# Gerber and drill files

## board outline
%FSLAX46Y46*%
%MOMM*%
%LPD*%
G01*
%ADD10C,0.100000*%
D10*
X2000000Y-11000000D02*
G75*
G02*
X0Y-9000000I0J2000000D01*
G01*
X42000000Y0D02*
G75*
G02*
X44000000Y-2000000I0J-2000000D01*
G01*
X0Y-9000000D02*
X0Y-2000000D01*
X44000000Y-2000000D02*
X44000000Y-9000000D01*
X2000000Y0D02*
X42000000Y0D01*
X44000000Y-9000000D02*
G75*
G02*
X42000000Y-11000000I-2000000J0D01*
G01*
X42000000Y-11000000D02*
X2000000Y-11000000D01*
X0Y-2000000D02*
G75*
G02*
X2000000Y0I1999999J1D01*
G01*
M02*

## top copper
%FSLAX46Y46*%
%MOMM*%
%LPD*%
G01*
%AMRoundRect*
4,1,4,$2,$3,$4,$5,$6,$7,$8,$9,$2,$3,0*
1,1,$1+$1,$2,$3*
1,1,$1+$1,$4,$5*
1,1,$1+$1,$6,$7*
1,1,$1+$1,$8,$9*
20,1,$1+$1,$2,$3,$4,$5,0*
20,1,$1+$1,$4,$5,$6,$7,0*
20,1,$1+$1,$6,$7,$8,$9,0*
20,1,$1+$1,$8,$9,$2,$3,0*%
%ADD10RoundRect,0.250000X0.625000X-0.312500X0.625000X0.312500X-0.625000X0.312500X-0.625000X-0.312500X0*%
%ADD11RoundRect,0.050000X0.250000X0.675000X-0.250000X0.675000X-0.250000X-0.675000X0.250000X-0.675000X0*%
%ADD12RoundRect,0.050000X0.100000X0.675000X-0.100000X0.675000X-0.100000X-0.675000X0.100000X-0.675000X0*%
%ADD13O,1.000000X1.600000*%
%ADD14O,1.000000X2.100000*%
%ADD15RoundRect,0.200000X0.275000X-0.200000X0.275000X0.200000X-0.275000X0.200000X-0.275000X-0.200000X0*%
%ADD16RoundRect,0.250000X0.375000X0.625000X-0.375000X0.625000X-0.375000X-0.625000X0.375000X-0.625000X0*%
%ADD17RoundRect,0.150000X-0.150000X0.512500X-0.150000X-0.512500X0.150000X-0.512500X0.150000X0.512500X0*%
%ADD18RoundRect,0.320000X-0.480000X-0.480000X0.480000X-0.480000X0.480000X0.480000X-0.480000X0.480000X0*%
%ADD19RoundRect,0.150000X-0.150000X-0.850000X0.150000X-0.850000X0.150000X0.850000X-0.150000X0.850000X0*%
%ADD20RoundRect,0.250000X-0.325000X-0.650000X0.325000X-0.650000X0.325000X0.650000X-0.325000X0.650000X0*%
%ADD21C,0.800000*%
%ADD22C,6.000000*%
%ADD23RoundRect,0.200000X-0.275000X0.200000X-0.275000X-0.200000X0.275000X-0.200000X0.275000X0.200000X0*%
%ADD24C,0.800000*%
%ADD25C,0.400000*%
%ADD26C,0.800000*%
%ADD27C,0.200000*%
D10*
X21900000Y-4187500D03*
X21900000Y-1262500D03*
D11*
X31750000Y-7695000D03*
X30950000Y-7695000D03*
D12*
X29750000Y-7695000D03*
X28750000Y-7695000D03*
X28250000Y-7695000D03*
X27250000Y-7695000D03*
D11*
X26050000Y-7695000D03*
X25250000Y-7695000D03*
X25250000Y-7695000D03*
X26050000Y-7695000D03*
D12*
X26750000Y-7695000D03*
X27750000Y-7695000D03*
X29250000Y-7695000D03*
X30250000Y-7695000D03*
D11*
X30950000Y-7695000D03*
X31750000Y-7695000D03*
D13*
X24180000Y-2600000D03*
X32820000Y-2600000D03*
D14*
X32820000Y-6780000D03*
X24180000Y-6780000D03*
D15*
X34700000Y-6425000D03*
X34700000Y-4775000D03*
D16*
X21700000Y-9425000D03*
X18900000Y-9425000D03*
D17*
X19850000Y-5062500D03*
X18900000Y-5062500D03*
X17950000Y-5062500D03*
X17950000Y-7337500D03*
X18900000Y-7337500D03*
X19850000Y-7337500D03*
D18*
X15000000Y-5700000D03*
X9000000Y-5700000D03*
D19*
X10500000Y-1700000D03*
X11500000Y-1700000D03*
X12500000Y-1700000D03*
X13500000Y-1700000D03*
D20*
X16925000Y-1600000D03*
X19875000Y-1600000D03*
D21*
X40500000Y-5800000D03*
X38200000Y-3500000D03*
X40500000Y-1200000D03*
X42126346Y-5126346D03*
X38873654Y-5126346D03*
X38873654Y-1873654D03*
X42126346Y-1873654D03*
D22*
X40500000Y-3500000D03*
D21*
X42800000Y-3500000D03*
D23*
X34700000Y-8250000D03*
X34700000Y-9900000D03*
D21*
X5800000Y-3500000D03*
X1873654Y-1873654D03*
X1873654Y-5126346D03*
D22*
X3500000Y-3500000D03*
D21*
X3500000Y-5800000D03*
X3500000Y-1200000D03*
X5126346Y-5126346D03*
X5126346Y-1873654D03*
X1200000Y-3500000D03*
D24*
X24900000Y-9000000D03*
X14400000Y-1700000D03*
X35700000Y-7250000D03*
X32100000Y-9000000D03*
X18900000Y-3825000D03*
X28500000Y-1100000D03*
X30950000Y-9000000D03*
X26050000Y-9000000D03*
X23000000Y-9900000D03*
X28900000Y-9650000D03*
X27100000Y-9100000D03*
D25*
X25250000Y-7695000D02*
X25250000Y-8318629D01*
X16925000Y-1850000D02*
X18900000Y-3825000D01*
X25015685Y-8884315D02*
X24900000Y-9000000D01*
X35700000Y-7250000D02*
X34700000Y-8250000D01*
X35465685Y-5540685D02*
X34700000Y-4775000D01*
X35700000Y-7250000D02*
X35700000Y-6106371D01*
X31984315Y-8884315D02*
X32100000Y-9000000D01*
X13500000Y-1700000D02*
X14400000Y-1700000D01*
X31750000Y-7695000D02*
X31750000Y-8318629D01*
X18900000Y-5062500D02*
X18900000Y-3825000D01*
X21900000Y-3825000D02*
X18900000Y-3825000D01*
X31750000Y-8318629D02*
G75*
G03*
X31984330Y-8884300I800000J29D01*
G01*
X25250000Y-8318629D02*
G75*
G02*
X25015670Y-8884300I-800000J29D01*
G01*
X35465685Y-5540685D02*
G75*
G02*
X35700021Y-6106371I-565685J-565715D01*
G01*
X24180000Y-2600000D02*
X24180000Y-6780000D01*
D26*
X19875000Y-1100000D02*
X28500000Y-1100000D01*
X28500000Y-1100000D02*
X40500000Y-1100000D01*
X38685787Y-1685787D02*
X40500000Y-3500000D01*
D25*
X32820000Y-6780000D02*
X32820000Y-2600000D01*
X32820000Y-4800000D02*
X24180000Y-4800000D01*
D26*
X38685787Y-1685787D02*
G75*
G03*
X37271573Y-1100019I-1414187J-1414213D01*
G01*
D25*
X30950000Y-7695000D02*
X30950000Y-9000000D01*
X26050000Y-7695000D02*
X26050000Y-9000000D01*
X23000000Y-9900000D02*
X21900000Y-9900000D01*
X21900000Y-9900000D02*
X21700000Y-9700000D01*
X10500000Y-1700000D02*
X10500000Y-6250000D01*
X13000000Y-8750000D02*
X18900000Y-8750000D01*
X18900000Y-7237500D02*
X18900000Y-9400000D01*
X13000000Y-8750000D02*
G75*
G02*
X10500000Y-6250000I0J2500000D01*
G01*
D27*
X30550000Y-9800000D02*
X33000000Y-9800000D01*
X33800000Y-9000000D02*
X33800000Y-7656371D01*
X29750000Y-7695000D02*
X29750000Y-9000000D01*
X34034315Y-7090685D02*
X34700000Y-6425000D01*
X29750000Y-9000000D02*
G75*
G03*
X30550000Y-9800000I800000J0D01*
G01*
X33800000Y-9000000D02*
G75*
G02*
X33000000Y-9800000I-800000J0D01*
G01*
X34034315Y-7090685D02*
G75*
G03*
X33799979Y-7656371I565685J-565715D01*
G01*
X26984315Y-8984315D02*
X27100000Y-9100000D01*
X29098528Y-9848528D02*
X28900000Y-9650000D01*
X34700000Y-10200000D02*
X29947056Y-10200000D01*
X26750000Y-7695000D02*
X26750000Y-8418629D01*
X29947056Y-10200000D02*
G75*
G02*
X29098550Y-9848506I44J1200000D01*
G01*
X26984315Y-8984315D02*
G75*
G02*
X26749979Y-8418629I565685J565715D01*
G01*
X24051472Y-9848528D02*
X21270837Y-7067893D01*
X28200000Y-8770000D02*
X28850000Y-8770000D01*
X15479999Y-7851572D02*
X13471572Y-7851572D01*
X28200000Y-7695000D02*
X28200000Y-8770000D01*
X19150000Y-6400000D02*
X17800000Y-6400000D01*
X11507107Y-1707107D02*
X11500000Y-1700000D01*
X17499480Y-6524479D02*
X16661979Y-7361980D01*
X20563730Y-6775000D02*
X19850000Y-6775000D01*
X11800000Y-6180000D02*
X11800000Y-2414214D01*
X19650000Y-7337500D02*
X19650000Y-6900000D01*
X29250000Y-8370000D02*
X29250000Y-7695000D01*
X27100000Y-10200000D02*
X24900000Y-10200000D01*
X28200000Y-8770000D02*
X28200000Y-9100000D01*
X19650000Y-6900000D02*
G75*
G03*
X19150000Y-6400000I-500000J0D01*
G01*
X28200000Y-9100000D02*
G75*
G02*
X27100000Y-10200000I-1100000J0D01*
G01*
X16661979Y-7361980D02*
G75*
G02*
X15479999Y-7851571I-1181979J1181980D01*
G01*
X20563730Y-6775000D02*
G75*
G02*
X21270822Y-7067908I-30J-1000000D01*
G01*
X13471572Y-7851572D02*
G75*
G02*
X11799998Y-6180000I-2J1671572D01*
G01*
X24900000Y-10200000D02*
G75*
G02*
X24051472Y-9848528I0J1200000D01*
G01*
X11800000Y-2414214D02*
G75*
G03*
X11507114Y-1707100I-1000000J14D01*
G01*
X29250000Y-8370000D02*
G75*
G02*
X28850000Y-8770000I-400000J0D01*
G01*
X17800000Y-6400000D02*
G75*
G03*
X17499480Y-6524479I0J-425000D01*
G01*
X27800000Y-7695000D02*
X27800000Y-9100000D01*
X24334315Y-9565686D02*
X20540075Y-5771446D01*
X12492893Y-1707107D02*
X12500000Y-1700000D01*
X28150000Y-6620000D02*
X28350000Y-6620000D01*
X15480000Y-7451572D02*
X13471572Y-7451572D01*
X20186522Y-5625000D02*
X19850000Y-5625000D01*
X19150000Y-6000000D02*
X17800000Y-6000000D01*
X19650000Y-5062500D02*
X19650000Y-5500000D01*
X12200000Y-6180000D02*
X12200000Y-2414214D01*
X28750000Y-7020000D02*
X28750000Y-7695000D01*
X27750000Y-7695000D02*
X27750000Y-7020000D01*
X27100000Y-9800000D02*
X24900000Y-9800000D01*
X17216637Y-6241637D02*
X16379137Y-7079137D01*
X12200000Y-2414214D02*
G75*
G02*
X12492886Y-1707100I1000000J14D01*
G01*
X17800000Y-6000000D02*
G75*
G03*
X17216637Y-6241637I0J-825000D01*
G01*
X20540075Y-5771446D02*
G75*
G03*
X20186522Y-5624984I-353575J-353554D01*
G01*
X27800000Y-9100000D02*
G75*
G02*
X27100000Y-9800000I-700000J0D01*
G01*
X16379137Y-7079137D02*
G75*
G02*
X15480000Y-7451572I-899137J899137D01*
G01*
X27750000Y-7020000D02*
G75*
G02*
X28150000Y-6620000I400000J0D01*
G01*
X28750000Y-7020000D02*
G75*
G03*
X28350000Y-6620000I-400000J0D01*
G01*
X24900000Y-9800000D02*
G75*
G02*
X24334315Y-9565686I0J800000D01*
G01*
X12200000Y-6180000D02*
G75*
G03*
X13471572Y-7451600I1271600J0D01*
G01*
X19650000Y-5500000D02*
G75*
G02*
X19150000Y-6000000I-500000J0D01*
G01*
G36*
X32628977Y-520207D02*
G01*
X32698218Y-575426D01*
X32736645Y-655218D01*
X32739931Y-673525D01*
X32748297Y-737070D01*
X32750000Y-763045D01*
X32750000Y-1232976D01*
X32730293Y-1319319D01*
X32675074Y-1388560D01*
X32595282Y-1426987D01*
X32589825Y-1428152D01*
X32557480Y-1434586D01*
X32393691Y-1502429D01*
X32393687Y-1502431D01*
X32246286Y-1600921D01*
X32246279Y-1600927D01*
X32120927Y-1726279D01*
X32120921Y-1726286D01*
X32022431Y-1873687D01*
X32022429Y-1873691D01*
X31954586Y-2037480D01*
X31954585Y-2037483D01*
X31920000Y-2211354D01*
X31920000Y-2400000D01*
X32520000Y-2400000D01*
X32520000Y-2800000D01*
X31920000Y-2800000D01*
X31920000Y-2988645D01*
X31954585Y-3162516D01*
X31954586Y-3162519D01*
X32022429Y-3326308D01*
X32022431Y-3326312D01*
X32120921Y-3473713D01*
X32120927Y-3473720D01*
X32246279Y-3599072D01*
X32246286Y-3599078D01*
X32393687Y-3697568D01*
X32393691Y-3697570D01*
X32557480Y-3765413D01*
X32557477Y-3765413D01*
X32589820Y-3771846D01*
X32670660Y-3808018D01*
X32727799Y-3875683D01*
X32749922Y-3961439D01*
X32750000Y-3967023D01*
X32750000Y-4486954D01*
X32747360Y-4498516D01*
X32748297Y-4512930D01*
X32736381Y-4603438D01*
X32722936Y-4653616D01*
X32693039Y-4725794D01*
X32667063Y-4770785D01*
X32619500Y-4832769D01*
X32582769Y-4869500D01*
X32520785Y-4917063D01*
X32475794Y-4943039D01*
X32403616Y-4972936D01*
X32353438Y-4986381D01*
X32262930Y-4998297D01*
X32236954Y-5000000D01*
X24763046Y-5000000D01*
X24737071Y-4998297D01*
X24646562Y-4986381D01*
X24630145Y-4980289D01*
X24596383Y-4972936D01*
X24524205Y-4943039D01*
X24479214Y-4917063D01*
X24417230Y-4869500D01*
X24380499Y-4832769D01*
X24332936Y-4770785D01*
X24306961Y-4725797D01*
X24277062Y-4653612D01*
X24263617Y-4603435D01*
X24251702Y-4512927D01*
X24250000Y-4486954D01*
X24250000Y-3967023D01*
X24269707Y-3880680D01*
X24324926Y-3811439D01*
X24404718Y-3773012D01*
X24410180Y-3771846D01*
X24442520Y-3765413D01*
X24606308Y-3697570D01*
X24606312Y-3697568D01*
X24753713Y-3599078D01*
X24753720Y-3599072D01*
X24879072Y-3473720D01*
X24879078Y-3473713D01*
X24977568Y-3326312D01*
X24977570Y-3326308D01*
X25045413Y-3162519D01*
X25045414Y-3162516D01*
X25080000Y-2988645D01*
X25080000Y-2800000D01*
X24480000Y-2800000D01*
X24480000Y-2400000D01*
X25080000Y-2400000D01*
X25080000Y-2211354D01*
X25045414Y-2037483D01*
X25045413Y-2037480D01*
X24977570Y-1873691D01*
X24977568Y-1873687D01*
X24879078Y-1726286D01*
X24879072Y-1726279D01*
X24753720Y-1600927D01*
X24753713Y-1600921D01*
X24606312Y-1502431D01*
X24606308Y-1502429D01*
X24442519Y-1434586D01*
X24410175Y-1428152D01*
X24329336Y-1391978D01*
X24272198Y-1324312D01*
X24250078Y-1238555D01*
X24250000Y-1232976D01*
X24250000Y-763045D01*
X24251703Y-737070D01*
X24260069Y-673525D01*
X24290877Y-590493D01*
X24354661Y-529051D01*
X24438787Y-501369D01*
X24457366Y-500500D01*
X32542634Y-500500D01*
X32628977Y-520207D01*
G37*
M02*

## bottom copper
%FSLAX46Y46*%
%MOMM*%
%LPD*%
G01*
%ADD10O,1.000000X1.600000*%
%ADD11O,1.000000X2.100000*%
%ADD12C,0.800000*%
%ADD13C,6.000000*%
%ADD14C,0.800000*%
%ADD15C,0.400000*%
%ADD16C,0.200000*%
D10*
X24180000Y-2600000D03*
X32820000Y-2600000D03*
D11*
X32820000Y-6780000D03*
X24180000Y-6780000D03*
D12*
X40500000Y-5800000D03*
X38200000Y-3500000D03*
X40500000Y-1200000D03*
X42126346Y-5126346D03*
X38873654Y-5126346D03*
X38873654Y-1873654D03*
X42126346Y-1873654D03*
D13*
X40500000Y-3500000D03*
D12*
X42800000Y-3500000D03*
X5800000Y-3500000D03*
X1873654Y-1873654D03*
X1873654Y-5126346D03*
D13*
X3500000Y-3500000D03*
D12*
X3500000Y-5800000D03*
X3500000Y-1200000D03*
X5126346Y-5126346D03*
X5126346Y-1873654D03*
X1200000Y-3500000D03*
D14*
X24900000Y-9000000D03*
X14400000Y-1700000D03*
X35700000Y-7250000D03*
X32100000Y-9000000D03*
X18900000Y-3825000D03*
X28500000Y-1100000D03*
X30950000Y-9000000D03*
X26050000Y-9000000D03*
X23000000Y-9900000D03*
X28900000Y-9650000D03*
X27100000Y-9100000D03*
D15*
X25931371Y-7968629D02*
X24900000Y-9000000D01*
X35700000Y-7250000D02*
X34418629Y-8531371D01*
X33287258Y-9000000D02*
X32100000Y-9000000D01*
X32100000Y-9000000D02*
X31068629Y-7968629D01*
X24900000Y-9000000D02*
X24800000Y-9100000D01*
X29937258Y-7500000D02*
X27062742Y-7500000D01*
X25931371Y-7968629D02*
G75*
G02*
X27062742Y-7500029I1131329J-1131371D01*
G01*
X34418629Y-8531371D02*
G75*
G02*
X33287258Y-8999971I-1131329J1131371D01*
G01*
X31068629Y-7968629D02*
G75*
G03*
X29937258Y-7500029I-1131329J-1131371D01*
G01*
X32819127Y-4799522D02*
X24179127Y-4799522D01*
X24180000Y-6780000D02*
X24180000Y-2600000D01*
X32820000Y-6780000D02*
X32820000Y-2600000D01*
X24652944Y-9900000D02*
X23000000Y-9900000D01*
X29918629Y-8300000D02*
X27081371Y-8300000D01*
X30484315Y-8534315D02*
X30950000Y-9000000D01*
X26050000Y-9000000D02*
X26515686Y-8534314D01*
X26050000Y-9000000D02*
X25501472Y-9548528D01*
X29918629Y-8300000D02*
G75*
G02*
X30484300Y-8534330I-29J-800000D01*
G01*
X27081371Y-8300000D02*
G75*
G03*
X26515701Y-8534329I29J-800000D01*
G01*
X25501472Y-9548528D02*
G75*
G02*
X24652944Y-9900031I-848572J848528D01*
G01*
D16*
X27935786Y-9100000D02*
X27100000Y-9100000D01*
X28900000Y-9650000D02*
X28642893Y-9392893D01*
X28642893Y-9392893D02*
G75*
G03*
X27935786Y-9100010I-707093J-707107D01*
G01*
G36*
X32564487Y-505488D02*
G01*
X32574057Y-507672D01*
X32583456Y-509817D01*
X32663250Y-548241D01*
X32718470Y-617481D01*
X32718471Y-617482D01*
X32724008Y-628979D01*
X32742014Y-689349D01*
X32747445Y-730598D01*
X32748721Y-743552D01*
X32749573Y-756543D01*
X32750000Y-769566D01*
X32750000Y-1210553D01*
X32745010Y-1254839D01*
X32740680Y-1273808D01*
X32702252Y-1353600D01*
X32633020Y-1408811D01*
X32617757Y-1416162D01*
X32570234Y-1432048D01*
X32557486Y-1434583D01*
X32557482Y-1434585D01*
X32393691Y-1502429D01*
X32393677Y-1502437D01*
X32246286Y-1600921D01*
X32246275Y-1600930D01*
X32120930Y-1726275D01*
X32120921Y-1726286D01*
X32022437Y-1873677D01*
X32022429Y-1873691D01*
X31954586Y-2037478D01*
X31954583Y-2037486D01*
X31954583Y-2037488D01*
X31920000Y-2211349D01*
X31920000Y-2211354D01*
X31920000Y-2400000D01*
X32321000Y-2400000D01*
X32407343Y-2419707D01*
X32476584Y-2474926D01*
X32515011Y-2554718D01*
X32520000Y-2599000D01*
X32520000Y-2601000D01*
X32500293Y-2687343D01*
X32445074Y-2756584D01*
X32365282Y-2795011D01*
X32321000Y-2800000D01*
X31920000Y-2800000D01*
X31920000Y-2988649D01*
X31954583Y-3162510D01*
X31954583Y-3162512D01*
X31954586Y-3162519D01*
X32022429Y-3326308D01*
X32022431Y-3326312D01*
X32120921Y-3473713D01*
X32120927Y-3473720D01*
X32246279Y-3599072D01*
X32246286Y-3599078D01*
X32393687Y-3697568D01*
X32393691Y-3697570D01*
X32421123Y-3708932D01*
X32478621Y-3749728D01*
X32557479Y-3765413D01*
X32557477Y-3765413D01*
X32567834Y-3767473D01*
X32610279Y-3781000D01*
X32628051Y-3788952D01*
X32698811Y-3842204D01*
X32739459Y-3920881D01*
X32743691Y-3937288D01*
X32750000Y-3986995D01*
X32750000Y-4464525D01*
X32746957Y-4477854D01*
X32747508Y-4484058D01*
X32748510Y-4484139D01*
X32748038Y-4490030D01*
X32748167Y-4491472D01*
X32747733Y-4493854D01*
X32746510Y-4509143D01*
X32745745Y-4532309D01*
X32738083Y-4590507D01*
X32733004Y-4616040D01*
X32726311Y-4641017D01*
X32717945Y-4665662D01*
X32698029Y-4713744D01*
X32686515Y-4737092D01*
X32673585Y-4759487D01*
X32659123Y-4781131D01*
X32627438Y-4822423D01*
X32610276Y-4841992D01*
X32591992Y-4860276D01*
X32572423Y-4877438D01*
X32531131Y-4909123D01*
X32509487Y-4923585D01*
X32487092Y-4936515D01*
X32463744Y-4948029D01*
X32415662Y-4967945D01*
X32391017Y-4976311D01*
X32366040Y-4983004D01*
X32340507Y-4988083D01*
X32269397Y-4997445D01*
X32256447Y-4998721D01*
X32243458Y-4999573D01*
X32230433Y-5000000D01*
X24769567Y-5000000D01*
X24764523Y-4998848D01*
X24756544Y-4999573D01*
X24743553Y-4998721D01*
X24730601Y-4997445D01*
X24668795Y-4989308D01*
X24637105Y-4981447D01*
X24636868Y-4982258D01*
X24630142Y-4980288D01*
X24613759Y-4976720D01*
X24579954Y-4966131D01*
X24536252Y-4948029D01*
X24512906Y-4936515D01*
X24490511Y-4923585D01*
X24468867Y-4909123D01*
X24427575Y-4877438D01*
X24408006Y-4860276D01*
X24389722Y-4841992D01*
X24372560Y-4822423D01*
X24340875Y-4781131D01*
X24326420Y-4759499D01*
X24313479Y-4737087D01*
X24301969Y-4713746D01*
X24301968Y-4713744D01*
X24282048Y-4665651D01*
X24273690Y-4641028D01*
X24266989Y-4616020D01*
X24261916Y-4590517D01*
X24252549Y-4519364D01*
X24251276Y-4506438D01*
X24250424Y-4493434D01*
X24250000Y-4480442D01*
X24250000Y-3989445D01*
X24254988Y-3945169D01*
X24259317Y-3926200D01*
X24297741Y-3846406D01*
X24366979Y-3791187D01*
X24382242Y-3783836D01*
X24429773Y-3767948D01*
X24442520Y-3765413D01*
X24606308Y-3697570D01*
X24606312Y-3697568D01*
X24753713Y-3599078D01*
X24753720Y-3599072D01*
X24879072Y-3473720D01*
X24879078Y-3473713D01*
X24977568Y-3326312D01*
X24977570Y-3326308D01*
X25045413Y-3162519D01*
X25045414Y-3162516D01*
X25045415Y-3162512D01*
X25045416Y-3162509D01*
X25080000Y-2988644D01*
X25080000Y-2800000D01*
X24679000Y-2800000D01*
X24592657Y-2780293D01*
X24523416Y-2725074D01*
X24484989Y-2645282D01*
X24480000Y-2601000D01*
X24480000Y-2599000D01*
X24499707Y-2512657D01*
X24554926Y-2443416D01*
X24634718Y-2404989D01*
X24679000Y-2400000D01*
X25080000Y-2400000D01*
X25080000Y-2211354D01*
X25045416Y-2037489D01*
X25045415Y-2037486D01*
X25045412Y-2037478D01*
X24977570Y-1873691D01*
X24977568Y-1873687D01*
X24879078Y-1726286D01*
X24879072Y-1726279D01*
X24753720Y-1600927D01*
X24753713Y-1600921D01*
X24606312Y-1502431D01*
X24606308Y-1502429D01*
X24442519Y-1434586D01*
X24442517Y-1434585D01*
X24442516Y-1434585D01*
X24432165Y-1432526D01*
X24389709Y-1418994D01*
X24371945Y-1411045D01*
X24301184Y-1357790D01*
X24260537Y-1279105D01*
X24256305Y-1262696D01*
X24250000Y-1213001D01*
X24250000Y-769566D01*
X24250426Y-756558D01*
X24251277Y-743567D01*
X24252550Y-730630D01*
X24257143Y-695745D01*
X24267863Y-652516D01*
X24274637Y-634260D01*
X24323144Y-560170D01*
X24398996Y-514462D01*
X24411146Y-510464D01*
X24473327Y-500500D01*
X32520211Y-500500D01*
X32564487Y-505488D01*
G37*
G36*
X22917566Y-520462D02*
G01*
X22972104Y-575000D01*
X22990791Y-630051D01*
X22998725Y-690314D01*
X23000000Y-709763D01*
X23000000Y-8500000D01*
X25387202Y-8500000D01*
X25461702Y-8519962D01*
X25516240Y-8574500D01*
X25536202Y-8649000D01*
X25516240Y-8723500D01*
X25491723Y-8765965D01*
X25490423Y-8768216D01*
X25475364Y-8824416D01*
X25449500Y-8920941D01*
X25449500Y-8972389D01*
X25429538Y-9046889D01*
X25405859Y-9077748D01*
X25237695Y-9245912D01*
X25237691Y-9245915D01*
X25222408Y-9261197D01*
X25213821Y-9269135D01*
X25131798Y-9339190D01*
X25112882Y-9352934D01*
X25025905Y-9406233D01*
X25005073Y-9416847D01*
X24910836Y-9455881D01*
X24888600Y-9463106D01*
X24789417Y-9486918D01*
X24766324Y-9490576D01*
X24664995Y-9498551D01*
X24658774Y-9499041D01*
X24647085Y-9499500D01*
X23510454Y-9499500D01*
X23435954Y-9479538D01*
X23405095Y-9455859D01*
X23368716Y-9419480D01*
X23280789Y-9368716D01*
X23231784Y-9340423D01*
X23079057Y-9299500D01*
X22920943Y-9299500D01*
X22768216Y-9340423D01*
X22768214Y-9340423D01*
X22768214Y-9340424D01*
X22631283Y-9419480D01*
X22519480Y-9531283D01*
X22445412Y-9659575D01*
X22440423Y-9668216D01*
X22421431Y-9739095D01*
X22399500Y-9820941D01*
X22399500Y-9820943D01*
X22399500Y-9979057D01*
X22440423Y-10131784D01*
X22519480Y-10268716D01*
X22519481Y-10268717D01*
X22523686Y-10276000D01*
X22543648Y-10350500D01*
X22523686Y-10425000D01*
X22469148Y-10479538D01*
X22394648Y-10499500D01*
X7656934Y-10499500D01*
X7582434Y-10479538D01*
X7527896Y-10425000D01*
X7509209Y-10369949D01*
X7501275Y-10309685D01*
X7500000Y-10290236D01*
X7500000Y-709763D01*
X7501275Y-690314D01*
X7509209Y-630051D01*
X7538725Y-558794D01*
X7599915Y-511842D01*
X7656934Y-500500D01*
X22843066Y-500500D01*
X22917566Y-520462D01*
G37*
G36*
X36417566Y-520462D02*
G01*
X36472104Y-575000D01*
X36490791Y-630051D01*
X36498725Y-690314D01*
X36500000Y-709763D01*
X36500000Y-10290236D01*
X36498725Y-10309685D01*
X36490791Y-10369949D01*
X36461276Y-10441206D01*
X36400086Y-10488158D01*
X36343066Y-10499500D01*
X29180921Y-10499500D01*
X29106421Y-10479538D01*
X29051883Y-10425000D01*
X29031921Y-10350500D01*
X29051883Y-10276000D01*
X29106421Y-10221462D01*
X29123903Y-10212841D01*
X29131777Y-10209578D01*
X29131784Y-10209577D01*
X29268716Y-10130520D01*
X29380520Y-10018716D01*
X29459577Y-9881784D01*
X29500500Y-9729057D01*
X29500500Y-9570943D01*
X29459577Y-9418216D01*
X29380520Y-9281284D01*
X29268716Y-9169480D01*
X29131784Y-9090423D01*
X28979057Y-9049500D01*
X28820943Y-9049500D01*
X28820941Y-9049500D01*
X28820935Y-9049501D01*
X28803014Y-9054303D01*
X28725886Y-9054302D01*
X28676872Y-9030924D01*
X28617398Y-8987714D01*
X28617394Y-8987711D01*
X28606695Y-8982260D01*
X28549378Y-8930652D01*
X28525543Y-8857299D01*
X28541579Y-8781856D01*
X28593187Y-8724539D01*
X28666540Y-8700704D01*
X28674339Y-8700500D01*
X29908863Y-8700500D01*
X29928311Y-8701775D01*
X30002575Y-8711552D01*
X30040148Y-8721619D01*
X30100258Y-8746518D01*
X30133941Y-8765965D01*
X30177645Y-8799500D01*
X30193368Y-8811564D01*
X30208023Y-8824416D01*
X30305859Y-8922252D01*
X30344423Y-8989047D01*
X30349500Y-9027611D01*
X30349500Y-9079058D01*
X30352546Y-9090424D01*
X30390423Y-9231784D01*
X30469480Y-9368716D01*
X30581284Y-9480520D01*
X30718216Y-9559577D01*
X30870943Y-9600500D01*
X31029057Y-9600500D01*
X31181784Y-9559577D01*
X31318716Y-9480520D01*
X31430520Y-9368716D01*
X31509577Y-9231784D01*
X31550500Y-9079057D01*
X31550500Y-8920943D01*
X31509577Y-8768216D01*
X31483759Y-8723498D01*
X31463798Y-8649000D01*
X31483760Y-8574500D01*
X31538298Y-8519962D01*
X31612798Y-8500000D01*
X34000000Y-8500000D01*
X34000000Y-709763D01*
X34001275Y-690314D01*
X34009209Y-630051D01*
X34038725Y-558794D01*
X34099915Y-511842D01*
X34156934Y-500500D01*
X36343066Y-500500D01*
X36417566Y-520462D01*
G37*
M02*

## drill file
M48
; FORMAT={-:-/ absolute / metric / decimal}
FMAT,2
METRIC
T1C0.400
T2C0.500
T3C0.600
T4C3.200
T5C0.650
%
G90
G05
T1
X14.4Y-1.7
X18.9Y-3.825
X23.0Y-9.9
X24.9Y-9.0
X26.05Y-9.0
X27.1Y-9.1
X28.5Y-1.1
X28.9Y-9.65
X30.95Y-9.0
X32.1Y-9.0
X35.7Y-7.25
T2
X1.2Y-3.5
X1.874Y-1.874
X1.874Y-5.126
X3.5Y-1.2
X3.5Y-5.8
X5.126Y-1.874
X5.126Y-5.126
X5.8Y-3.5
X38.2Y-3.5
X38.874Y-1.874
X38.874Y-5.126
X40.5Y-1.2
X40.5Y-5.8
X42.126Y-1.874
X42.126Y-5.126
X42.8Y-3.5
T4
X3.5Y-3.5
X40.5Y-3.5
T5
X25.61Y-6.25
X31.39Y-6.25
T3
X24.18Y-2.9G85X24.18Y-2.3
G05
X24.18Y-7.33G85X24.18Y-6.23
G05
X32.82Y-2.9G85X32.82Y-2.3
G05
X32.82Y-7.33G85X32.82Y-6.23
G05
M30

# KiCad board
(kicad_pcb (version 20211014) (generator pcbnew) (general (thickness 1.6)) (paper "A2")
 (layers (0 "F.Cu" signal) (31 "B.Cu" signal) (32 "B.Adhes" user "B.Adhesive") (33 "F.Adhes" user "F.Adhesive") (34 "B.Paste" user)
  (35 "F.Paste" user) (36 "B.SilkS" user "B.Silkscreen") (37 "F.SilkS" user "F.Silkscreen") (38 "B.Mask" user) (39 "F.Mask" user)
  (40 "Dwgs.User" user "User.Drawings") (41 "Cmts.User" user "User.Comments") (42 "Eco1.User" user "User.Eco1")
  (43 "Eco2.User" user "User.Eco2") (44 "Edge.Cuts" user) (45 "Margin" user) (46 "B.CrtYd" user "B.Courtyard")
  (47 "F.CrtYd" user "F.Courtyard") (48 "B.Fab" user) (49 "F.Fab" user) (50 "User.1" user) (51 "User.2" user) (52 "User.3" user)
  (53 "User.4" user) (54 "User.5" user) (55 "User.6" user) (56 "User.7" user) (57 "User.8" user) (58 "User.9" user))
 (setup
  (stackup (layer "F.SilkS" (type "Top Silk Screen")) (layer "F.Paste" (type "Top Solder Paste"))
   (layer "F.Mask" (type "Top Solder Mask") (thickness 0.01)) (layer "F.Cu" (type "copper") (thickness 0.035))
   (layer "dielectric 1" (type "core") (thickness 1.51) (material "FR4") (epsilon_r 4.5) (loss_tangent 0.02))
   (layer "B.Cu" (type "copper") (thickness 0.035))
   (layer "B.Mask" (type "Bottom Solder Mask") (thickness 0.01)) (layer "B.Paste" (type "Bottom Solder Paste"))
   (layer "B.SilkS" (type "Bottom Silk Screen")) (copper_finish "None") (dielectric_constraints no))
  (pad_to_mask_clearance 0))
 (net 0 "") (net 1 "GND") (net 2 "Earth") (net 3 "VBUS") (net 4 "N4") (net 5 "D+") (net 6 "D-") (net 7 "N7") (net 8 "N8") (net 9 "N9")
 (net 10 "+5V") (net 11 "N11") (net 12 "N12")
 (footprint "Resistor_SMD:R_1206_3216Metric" (layer "F.Cu") (at 21.9 2.725 90)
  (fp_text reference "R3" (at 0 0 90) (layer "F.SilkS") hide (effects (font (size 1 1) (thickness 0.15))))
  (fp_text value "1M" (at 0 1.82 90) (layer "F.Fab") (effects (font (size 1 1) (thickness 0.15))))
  (pad "1" smd roundrect (at -1.4625 0 90) (size 1.125 1.75) (layers "F.Cu" "F.Paste" "F.Mask") (roundrect_rratio 0.2222222222)
   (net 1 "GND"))
  (pad "2" smd roundrect (at 1.4625 0 90) (size 1.125 1.75) (layers "F.Cu" "F.Paste" "F.Mask") (roundrect_rratio 0.2222222222)
   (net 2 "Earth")))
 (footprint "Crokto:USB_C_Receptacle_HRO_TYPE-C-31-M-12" (layer "F.Cu") (at 28.5 3.65 180)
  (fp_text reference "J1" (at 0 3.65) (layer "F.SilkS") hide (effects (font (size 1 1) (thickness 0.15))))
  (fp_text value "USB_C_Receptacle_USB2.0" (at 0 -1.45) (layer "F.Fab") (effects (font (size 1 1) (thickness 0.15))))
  (pad "" np_thru_hole circle (at -2.89 -2.6 180) (size 0.65 0.65) (drill 0.65) (layers *.Cu *.Mask))
  (pad "" np_thru_hole circle (at 2.89 -2.6 180) (size 0.65 0.65) (drill 0.65) (layers *.Cu *.Mask))
  (pad "A1" smd roundrect (at -3.25 -4.045 180) (size 0.6 1.45) (layers "F.Cu" "F.Paste" "F.Mask") (roundrect_rratio 0.08333333333)
   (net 1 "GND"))
  (pad "A4" smd roundrect (at -2.45 -4.045 180) (size 0.6 1.45) (layers "F.Cu" "F.Paste" "F.Mask") (roundrect_rratio 0.08333333333)
   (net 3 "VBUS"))
  (pad "A5" smd roundrect (at -1.25 -4.045 180) (size 0.3 1.45) (layers "F.Cu" "F.Paste" "F.Mask") (roundrect_rratio 0.1666666667)
   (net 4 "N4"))
  (pad "A6" smd roundrect (at -0.25 -4.045 180) (size 0.3 1.45) (layers "F.Cu" "F.Paste" "F.Mask") (roundrect_rratio 0.1666666667)
   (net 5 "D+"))
  (pad "A7" smd roundrect (at 0.25 -4.045 180) (size 0.3 1.45) (layers "F.Cu" "F.Paste" "F.Mask") (roundrect_rratio 0.1666666667)
   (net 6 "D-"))
  (pad "A8" smd roundrect (at 1.25 -4.045 180) (size 0.3 1.45) (layers "F.Cu" "F.Paste" "F.Mask") (roundrect_rratio 0.1666666667)
   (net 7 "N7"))
  (pad "A9" smd roundrect (at 2.45 -4.045 180) (size 0.6 1.45) (layers "F.Cu" "F.Paste" "F.Mask") (roundrect_rratio 0.08333333333)
   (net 3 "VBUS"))
  (pad "A12" smd roundrect (at 3.25 -4.045 180) (size 0.6 1.45) (layers "F.Cu" "F.Paste" "F.Mask") (roundrect_rratio 0.08333333333)
   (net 1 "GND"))
  (pad "B1" smd roundrect (at 3.25 -4.045 180) (size 0.6 1.45) (layers "F.Cu" "F.Paste" "F.Mask") (roundrect_rratio 0.08333333333)
   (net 1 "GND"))
  (pad "B4" smd roundrect (at 2.45 -4.045 180) (size 0.6 1.45) (layers "F.Cu" "F.Paste" "F.Mask") (roundrect_rratio 0.08333333333)
   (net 3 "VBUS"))
  (pad "B5" smd roundrect (at 1.75 -4.045 180) (size 0.3 1.45) (layers "F.Cu" "F.Paste" "F.Mask") (roundrect_rratio 0.1666666667)
   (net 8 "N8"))
  (pad "B6" smd roundrect (at 0.75 -4.045 180) (size 0.3 1.45) (layers "F.Cu" "F.Paste" "F.Mask") (roundrect_rratio 0.1666666667)
   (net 5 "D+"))
  (pad "B7" smd roundrect (at -0.75 -4.045 180) (size 0.3 1.45) (layers "F.Cu" "F.Paste" "F.Mask") (roundrect_rratio 0.1666666667)
   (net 6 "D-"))
  (pad "B8" smd roundrect (at -1.75 -4.045 180) (size 0.3 1.45) (layers "F.Cu" "F.Paste" "F.Mask") (roundrect_rratio 0.1666666667)
   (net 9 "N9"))
  (pad "B9" smd roundrect (at -2.45 -4.045 180) (size 0.6 1.45) (layers "F.Cu" "F.Paste" "F.Mask") (roundrect_rratio 0.08333333333)
   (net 3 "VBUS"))
  (pad "B12" smd roundrect (at -3.25 -4.045 180) (size 0.6 1.45) (layers "F.Cu" "F.Paste" "F.Mask") (roundrect_rratio 0.08333333333)
   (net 1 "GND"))
  (pad "S1" thru_hole oval (at 4.32 1.05 180) (size 1 1.6) (drill oval 0.6 1.2) (layers *.Cu *.Mask) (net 2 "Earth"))
  (pad "S1" thru_hole oval (at -4.32 1.05 180) (size 1 1.6) (drill oval 0.6 1.2) (layers *.Cu *.Mask) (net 2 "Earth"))
  (pad "S1" thru_hole oval (at -4.32 -3.13 180) (size 1 2.1) (drill oval 0.6 1.7) (layers *.Cu *.Mask) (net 2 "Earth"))
  (pad "S1" thru_hole oval (at 4.32 -3.13 180) (size 1 2.1) (drill oval 0.6 1.7) (layers *.Cu *.Mask) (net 2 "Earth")))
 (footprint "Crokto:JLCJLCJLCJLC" (layer "F.Cu") (at 84.5 4.6 180)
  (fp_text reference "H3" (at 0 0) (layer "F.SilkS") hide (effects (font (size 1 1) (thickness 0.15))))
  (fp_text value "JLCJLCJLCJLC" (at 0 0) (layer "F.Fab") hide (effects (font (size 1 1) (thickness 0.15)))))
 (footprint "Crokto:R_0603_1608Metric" (layer "F.Cu") (at 34.7 5.6 90)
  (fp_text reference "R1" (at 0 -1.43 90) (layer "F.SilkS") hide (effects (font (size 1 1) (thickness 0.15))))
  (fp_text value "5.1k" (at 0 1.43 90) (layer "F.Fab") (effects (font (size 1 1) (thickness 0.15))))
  (pad "1" smd roundrect (at -0.825 0 90) (size 0.8 0.95) (layers "F.Cu" "F.Paste" "F.Mask") (roundrect_rratio 0.25) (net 4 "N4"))
  (pad "2" smd roundrect (at 0.825 0 90) (size 0.8 0.95) (layers "F.Cu" "F.Paste" "F.Mask") (roundrect_rratio 0.25) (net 1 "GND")))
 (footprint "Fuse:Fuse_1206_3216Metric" (layer "F.Cu") (at 20.3 9.425 180)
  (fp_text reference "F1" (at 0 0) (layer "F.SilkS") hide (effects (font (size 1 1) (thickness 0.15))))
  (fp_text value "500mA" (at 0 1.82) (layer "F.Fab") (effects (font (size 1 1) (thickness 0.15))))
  (pad "1" smd roundrect (at -1.4 0 180) (size 1.25 1.75) (layers "F.Cu" "F.Paste" "F.Mask") (roundrect_rratio 0.2) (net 3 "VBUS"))
  (pad "2" smd roundrect (at 1.4 0 180) (size 1.25 1.75) (layers "F.Cu" "F.Paste" "F.Mask") (roundrect_rratio 0.2) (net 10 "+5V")))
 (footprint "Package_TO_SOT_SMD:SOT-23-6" (layer "F.Cu") (at 18.9 6.2 -90)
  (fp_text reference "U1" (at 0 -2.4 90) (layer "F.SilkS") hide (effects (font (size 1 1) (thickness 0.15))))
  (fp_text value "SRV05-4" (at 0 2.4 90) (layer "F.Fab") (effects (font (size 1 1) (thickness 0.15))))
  (pad "1" smd roundrect (at -1.1375 -0.95 270) (size 1.325 0.6) (layers "F.Cu" "F.Paste" "F.Mask") (roundrect_rratio 0.25) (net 5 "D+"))
  (pad "2" smd roundrect (at -1.1375 0 270) (size 1.325 0.6) (layers "F.Cu" "F.Paste" "F.Mask") (roundrect_rratio 0.25) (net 1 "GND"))
  (pad "3" smd roundrect (at -1.1375 0.95 270) (size 1.325 0.6) (layers "F.Cu" "F.Paste" "F.Mask") (roundrect_rratio 0.25) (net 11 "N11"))
  (pad "4" smd roundrect (at 1.1375 0.95 270) (size 1.325 0.6) (layers "F.Cu" "F.Paste" "F.Mask") (roundrect_rratio 0.25) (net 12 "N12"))
  (pad "5" smd roundrect (at 1.1375 0 270) (size 1.325 0.6) (layers "F.Cu" "F.Paste" "F.Mask") (roundrect_rratio 0.25) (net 10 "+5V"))
  (pad "6" smd roundrect (at 1.1375 -0.95 270) (size 1.325 0.6) (layers "F.Cu" "F.Paste" "F.Mask") (roundrect_rratio 0.25) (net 6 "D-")))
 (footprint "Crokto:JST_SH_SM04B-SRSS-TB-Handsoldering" (layer "F.Cu") (at 12 3.925)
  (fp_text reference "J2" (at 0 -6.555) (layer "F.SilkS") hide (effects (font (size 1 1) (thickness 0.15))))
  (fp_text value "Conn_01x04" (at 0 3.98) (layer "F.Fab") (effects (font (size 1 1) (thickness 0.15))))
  (pad "" smd roundrect (at 3 1.775) (size 1.6 1.6) (layers "F.Cu" "F.Paste" "F.Mask") (roundrect_rratio 0.2))
  (pad "" smd roundrect (at -3 1.775) (size 1.6 1.6) (layers "F.Cu" "F.Paste" "F.Mask") (roundrect_rratio 0.2))
  (pad "1" smd roundrect (at -1.5 -2.225) (size 0.6 2) (layers "F.Cu" "F.Paste" "F.Mask") (roundrect_rratio 0.25) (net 10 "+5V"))
  (pad "2" smd roundrect (at -0.5 -2.225) (size 0.6 2) (layers "F.Cu" "F.Paste" "F.Mask") (roundrect_rratio 0.25) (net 6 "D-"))
  (pad "3" smd roundrect (at 0.5 -2.225) (size 0.6 2) (layers "F.Cu" "F.Paste" "F.Mask") (roundrect_rratio 0.25) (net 5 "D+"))
  (pad "4" smd roundrect (at 1.5 -2.225) (size 0.6 2) (layers "F.Cu" "F.Paste" "F.Mask") (roundrect_rratio 0.25) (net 1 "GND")))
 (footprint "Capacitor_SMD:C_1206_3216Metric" (layer "F.Cu") (at 18.4 1.6)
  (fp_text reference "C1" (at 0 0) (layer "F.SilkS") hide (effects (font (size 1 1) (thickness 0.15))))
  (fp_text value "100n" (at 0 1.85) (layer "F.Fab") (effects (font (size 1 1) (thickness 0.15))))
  (pad "1" smd roundrect (at -1.475 0) (size 1.15 1.8) (layers "F.Cu" "F.Paste" "F.Mask") (roundrect_rratio 0.2173913043) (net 1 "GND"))
  (pad "2" smd roundrect (at 1.475 0) (size 1.15 1.8) (layers "F.Cu" "F.Paste" "F.Mask") (roundrect_rratio 0.2173913043) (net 2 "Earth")))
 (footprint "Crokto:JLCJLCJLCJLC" (layer "F.Cu") (at 28.5 4.6 180)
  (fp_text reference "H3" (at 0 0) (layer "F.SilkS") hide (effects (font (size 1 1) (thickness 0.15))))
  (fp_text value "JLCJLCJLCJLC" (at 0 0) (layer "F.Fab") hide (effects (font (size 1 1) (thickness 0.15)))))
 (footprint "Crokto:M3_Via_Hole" (layer "F.Cu") (at 40.5 3.5)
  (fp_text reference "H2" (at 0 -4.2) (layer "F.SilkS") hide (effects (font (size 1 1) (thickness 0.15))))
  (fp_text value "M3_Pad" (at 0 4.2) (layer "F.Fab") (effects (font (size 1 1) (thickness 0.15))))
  (pad "1" thru_hole circle locked (at 0 2.3) (size 0.8 0.8) (drill 0.5) (layers *.Cu *.Mask) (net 2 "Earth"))
  (pad "1" thru_hole circle locked (at -2.3 0) (size 0.8 0.8) (drill 0.5) (layers *.Cu *.Mask) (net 2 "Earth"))
  (pad "1" thru_hole circle locked (at 0 -2.3) (size 0.8 0.8) (drill 0.5) (layers *.Cu *.Mask) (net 2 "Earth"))
  (pad "1" thru_hole circle locked (at 1.626346 1.626346) (size 0.8 0.8) (drill 0.5) (layers *.Cu *.Mask) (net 2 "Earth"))
  (pad "1" thru_hole circle locked (at -1.626346 1.626346) (size 0.8 0.8) (drill 0.5) (layers *.Cu *.Mask) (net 2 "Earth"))
  (pad "1" thru_hole circle locked (at -1.626346 -1.626346) (size 0.8 0.8) (drill 0.5) (layers *.Cu *.Mask) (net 2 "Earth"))
  (pad "1" thru_hole circle locked (at 1.626346 -1.626346) (size 0.8 0.8) (drill 0.5) (layers *.Cu *.Mask) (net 2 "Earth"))
  (pad "1" thru_hole circle locked (at 0 0) (size 6 6) (drill 3.2) (layers *.Cu *.Mask) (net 2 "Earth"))
  (pad "1" thru_hole circle locked (at 2.3 0) (size 0.8 0.8) (drill 0.5) (layers *.Cu *.Mask) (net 2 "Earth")))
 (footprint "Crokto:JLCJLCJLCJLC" (layer "F.Cu") (at 28.5 19.1 180)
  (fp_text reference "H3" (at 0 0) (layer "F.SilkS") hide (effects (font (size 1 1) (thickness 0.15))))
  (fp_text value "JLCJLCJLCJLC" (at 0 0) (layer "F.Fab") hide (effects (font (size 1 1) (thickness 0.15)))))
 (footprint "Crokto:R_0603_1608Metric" (layer "F.Cu") (at 34.7 9.075 -90)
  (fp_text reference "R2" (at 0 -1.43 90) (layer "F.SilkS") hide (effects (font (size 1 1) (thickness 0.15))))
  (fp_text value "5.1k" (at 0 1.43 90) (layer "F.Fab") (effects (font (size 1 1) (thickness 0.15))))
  (pad "1" smd roundrect (at -0.825 0 270) (size 0.8 0.95) (layers "F.Cu" "F.Paste" "F.Mask") (roundrect_rratio 0.25) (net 1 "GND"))
  (pad "2" smd roundrect (at 0.825 0 270) (size 0.8 0.95) (layers "F.Cu" "F.Paste" "F.Mask") (roundrect_rratio 0.25) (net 8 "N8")))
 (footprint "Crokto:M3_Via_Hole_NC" (layer "B.Cu") (at 3.5 3.5 180)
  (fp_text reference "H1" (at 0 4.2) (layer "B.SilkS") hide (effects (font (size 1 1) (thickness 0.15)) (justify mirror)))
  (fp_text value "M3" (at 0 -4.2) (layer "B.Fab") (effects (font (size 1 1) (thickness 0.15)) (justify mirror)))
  (pad "" thru_hole circle (at -2.3 0 180) (size 0.8 0.8) (drill 0.5) (layers *.Cu "B.Mask"))
  (pad "" thru_hole circle (at 1.626346 1.626346 180) (size 0.8 0.8) (drill 0.5) (layers *.Cu "B.Mask"))
  (pad "" thru_hole circle (at 1.626346 -1.626346 180) (size 0.8 0.8) (drill 0.5) (layers *.Cu "B.Mask"))
  (pad "" thru_hole circle (at 0 0 180) (size 6 6) (drill 3.2) (layers *.Cu "B.Mask"))
  (pad "" thru_hole circle (at 0 -2.3 180) (size 0.8 0.8) (drill 0.5) (layers *.Cu "B.Mask"))
  (pad "" thru_hole circle (at 0 2.3 180) (size 0.8 0.8) (drill 0.5) (layers *.Cu "B.Mask"))
  (pad "" thru_hole circle (at -1.626346 -1.626346 180) (size 0.8 0.8) (drill 0.5) (layers *.Cu "B.Mask"))
  (pad "" thru_hole circle (at -1.626346 1.626346 180) (size 0.8 0.8) (drill 0.5) (layers *.Cu "B.Mask"))
  (pad "" thru_hole circle (at 2.3 0 180) (size 0.8 0.8) (drill 0.5) (layers *.Cu "B.Mask")))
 (gr_arc (start 2 11) (mid 0.585786 10.414214) (end 0 9) (layer "Edge.Cuts") (width 0.1))
 (gr_arc (start 42 0) (mid 43.414214 0.585786) (end 44 2) (layer "Edge.Cuts") (width 0.1))
 (gr_line (start 0 9) (end 0 2) (layer "Edge.Cuts") (width 0.1))
 (gr_line (start 44 2) (end 44 9) (layer "Edge.Cuts") (width 0.1))
 (gr_line (start 2 0) (end 42 0) (layer "Edge.Cuts") (width 0.1))
 (gr_arc (start 44 9) (mid 43.414214 10.414214) (end 42 11) (layer "Edge.Cuts") (width 0.1))
 (gr_line (start 42 11) (end 2 11) (layer "Edge.Cuts") (width 0.1))
 (gr_arc (start 0 2) (mid 0.585786 0.585786) (end 2 0) (layer "Edge.Cuts") (width 0.1))
 (segment (start 25.25 7.695) (end 25.25 8.318629) (width 0.4) (layer "F.Cu") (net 1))
 (segment (start 16.925 1.85) (end 18.9 3.825) (width 0.4) (layer "F.Cu") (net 1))
 (segment (start 25.015685 8.884315) (end 24.9 9) (width 0.4) (layer "F.Cu") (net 1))
 (segment (start 35.7 7.25) (end 34.7 8.25) (width 0.4) (layer "F.Cu") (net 1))
 (segment (start 35.465685 5.540685) (end 34.7 4.775) (width 0.4) (layer "F.Cu") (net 1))
 (segment (start 35.7 7.25) (end 35.7 6.106371) (width 0.4) (layer "F.Cu") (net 1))
 (segment (start 31.984315 8.884315) (end 32.1 9) (width 0.4) (layer "F.Cu") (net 1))
 (segment (start 13.5 1.7) (end 14.4 1.7) (width 0.4) (layer "F.Cu") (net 1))
 (segment (start 31.75 7.695) (end 31.75 8.318629) (width 0.4) (layer "F.Cu") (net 1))
 (segment (start 18.9 5.0625) (end 18.9 3.825) (width 0.4) (layer "F.Cu") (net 1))
 (segment (start 21.9 3.825) (end 18.9 3.825) (width 0.4) (layer "F.Cu") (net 1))
 (via (at 24.9 9) (size 0.8) (drill 0.4) (layers "F.Cu" "B.Cu") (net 1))
 (via (at 14.4 1.7) (size 0.8) (drill 0.4) (layers "F.Cu" "B.Cu") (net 1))
 (via (at 35.7 7.25) (size 0.8) (drill 0.4) (layers "F.Cu" "B.Cu") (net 1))
 (via (at 32.1 9) (size 0.8) (drill 0.4) (layers "F.Cu" "B.Cu") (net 1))
 (via (at 18.9 3.825) (size 0.8) (drill 0.4) (layers "F.Cu" "B.Cu") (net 1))
 (arc (start 31.75 8.318629) (mid 31.810897 8.624776) (end 31.984315 8.884315) (width 0.4) (layer "F.Cu") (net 1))
 (arc (start 25.25 8.318629) (mid 25.189103 8.624776) (end 25.015685 8.884315) (width 0.4) (layer "F.Cu") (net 1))
 (arc (start 35.465685 5.540685) (mid 35.639104 5.800224) (end 35.7 6.106371) (width 0.4) (layer "F.Cu") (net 1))
 (segment (start 25.931371 7.968629) (end 24.9 9) (width 0.4) (layer "B.Cu") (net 1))
 (segment (start 35.7 7.25) (end 34.418629 8.531371) (width 0.4) (layer "B.Cu") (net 1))
 (segment (start 33.287258 9) (end 32.1 9) (width 0.4) (layer "B.Cu") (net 1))
 (segment (start 32.1 9) (end 31.068629 7.968629) (width 0.4) (layer "B.Cu") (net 1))
 (segment (start 24.9 9) (end 24.8 9.1) (width 0.4) (layer "B.Cu") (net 1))
 (segment (start 29.937258 7.5) (end 27.062742 7.5) (width 0.4) (layer "B.Cu") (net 1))
 (arc (start 25.931371 7.968629) (mid 26.450448 7.621793) (end 27.062742 7.5) (width 0.4) (layer "B.Cu") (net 1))
 (arc (start 34.418629 8.531371) (mid 33.899552 8.878207) (end 33.287258 9) (width 0.4) (layer "B.Cu") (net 1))
 (arc (start 31.068629 7.968629) (mid 30.549552 7.621793) (end 29.937258 7.5) (width 0.4) (layer "B.Cu") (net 1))
 (segment (start 24.18 2.6) (end 24.18 6.78) (width 0.4) (layer "F.Cu") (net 2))
 (segment (start 19.875 1.1) (end 28.5 1.1) (width 0.8) (layer "F.Cu") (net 2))
 (segment (start 28.5 1.1) (end 40.5 1.1) (width 0.8) (layer "F.Cu") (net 2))
 (segment (start 38.685787 1.685787) (end 40.5 3.5) (width 0.8) (layer "F.Cu") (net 2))
 (segment (start 32.82 6.78) (end 32.82 2.6) (width 0.4) (layer "F.Cu") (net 2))
 (segment (start 32.82 4.8) (end 24.18 4.8) (width 0.4) (layer "F.Cu") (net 2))
 (via (at 28.5 1.1) (size 0.8) (drill 0.4) (layers "F.Cu" "B.Cu") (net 2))
 (arc (start 38.685787 1.685787) (mid 38.03694 1.252241) (end 37.271573 1.1) (width 0.8) (layer "F.Cu") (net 2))
 (segment (start 32.819127 4.799522) (end 24.179127 4.799522) (width 0.4) (layer "B.Cu") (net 2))
 (segment (start 24.18 6.78) (end 24.18 2.6) (width 0.4) (layer "B.Cu") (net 2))
 (segment (start 32.82 6.78) (end 32.82 2.6) (width 0.4) (layer "B.Cu") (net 2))
 (segment (start 30.95 7.695) (end 30.95 9) (width 0.4) (layer "F.Cu") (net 3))
 (segment (start 26.05 7.695) (end 26.05 9) (width 0.4) (layer "F.Cu") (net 3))
 (segment (start 23 9.9) (end 21.9 9.9) (width 0.4) (layer "F.Cu") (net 3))
 (segment (start 21.9 9.9) (end 21.7 9.7) (width 0.4) (layer "F.Cu") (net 3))
 (via (at 30.95 9) (size 0.8) (drill 0.4) (layers "F.Cu" "B.Cu") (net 3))
 (via (at 26.05 9) (size 0.8) (drill 0.4) (layers "F.Cu" "B.Cu") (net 3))
 (via (at 23 9.9) (size 0.8) (drill 0.4) (layers "F.Cu" "B.Cu") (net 3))
 (segment (start 24.652944 9.9) (end 23 9.9) (width 0.4) (layer "B.Cu") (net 3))
 (segment (start 29.918629 8.3) (end 27.081371 8.3) (width 0.4) (layer "B.Cu") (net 3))
 (segment (start 30.484315 8.534315) (end 30.95 9) (width 0.4) (layer "B.Cu") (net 3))
 (segment (start 26.05 9) (end 26.515686 8.534314) (width 0.4) (layer "B.Cu") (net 3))
 (segment (start 26.05 9) (end 25.501472 9.548528) (width 0.4) (layer "B.Cu") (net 3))
 (arc (start 29.918629 8.3) (mid 30.224776 8.360897) (end 30.484315 8.534315) (width 0.4) (layer "B.Cu") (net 3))
 (arc (start 27.081371 8.3) (mid 26.775225 8.360896) (end 26.515686 8.534314) (width 0.4) (layer "B.Cu") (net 3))
 (arc (start 25.501472 9.548528) (mid 25.112164 9.808655) (end 24.652944 9.9) (width 0.4) (layer "B.Cu") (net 3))
 (segment (start 10.5 1.7) (end 10.5 6.25) (width 0.4) (layer "F.Cu") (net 10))
 (segment (start 13 8.75) (end 18.9 8.75) (width 0.4) (layer "F.Cu") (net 10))
 (segment (start 18.9 7.2375) (end 18.9 9.4) (width 0.4) (layer "F.Cu") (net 10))
 (arc (start 13 8.75) (mid 11.232233 8.017767) (end 10.5 6.25) (width 0.4) (layer "F.Cu") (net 10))
 (segment (start 30.55 9.8) (end 33 9.8) (width 0.2) (layer "F.Cu") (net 4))
 (segment (start 33.8 9) (end 33.8 7.656371) (width 0.2) (layer "F.Cu") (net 4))
 (segment (start 29.75 7.695) (end 29.75 9) (width 0.2) (layer "F.Cu") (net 4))
 (segment (start 34.034315 7.090685) (end 34.7 6.425) (width 0.2) (layer "F.Cu") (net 4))
 (arc (start 29.75 9) (mid 29.984315 9.565685) (end 30.55 9.8) (width 0.2) (layer "F.Cu") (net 4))
 (arc (start 33.8 9) (mid 33.565685 9.565685) (end 33 9.8) (width 0.2) (layer "F.Cu") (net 4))
 (arc (start 34.034315 7.090685) (mid 33.860896 7.350224) (end 33.8 7.656371) (width 0.2) (layer "F.Cu") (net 4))
 (segment (start 26.984315 8.984315) (end 27.1 9.1) (width 0.2) (layer "F.Cu") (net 8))
 (segment (start 29.098528 9.848528) (end 28.9 9.65) (width 0.2) (layer "F.Cu") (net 8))
 (segment (start 34.7 10.2) (end 29.947056 10.2) (width 0.2) (layer "F.Cu") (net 8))
 (segment (start 26.75 7.695) (end 26.75 8.418629) (width 0.2) (layer "F.Cu") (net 8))
 (via (at 28.9 9.65) (size 0.8) (drill 0.4) (layers "F.Cu" "B.Cu") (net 8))
 (via (at 27.1 9.1) (size 0.8) (drill 0.4) (layers "F.Cu" "B.Cu") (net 8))
 (arc (start 29.947056 10.2) (mid 29.487836 10.108655) (end 29.098528 9.848528) (width 0.2) (layer "F.Cu") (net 8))
 (arc (start 26.984315 8.984315) (mid 26.810896 8.724776) (end 26.75 8.418629) (width 0.2) (layer "F.Cu") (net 8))
 (segment (start 27.935786 9.1) (end 27.1 9.1) (width 0.2) (layer "B.Cu") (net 8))
 (segment (start 28.9 9.65) (end 28.642893 9.392893) (width 0.2) (layer "B.Cu") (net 8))
 (arc (start 28.642893 9.392893) (mid 28.31847 9.17612) (end 27.935786 9.1) (width 0.2) (layer "B.Cu") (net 8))
 (segment (start 24.051472 9.848528) (end 21.270837 7.067893) (width 0.2) (layer "F.Cu") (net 6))
 (segment (start 28.2 8.77) (end 28.85 8.77) (width 0.2) (layer "F.Cu") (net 6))
 (segment (start 15.479999 7.851572) (end 13.471572 7.851572) (width 0.2) (layer "F.Cu") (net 6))
 (segment (start 28.2 7.695) (end 28.2 8.77) (width 0.2) (layer "F.Cu") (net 6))
 (segment (start 19.15 6.4) (end 17.8 6.4) (width 0.2) (layer "F.Cu") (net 6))
 (segment (start 11.507107 1.707107) (end 11.5 1.7) (width 0.2) (layer "F.Cu") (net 6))
 (segment (start 17.49948 6.524479) (end 16.661979 7.36198) (width 0.2) (layer "F.Cu") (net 6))
 (segment (start 20.56373 6.775) (end 19.85 6.775) (width 0.2) (layer "F.Cu") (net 6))
 (segment (start 11.8 6.18) (end 11.8 2.414214) (width 0.2) (layer "F.Cu") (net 6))
 (segment (start 19.65 7.3375) (end 19.65 6.9) (width 0.2) (layer "F.Cu") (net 6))
 (segment (start 29.25 8.37) (end 29.25 7.695) (width 0.2) (layer "F.Cu") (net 6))
 (segment (start 27.1 10.2) (end 24.9 10.2) (width 0.2) (layer "F.Cu") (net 6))
 (segment (start 28.2 8.77) (end 28.2 9.1) (width 0.2) (layer "F.Cu") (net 6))
 (arc (start 19.65 6.9) (mid 19.503553 6.546447) (end 19.15 6.4) (width 0.2) (layer "F.Cu") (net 6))
 (arc (start 28.2 9.1) (mid 27.877817 9.877817) (end 27.1 10.2) (width 0.2) (layer "F.Cu") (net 6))
 (arc (start 16.661979 7.36198) (mid 16.119682 7.724331) (end 15.479999 7.851572) (width 0.2) (layer "F.Cu") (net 6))
 (arc (start 20.56373 6.775) (mid 20.946413 6.85112) (end 21.270837 7.067893) (width 0.2) (layer "F.Cu") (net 6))
 (arc (start 13.471572 7.851572) (mid 12.289592 7.36198) (end 11.8 6.18) (width 0.2) (layer "F.Cu") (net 6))
 (arc (start 24.9 10.2) (mid 24.44078 10.108655) (end 24.051472 9.848528) (width 0.2) (layer "F.Cu") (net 6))
 (arc (start 11.8 2.414214) (mid 11.72388 2.031531) (end 11.507107 1.707107) (width 0.2) (layer "F.Cu") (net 6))
 (arc (start 29.25 8.37) (mid 29.132843 8.652843) (end 28.85 8.77) (width 0.2) (layer "F.Cu") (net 6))
 (arc (start 17.8 6.4) (mid 17.63736 6.432351) (end 17.49948 6.524479) (width 0.2) (layer "F.Cu") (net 6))
 (segment (start 27.8 7.695) (end 27.8 9.1) (width 0.2) (layer "F.Cu") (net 5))
 (segment (start 24.334315 9.565686) (end 20.540075 5.771446) (width 0.2) (layer "F.Cu") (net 5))
 (segment (start 12.492893 1.707107) (end 12.5 1.7) (width 0.2) (layer "F.Cu") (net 5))
 (segment (start 28.15 6.62) (end 28.35 6.62) (width 0.2) (layer "F.Cu") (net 5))
 (segment (start 15.48 7.451572) (end 13.471572 7.451572) (width 0.2) (layer "F.Cu") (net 5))
 (segment (start 20.186522 5.625) (end 19.85 5.625) (width 0.2) (layer "F.Cu") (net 5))
 (segment (start 19.15 6) (end 17.8 6) (width 0.2) (layer "F.Cu") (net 5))
 (segment (start 19.65 5.0625) (end 19.65 5.5) (width 0.2) (layer "F.Cu") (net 5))
 (segment (start 12.2 6.18) (end 12.2 2.414214) (width 0.2) (layer "F.Cu") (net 5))
 (segment (start 28.75 7.02) (end 28.75 7.695) (width 0.2) (layer "F.Cu") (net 5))
 (segment (start 27.75 7.695) (end 27.75 7.02) (width 0.2) (layer "F.Cu") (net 5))
 (segment (start 27.1 9.8) (end 24.9 9.8) (width 0.2) (layer "F.Cu") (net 5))
 (segment (start 17.216637 6.241637) (end 16.379137 7.079137) (width 0.2) (layer "F.Cu") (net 5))
 (arc (start 12.2 2.414214) (mid 12.27612 2.031531) (end 12.492893 1.707107) (width 0.2) (layer "F.Cu") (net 5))
 (arc (start 17.8 6) (mid 17.484286 6.0628) (end 17.216637 6.241637) (width 0.2) (layer "F.Cu") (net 5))
 (arc (start 20.540075 5.771446) (mid 20.377863 5.66306) (end 20.186522 5.625) (width 0.2) (layer "F.Cu") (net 5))
 (arc (start 27.8 9.1) (mid 27.594975 9.594975) (end 27.1 9.8) (width 0.2) (layer "F.Cu") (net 5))
 (arc (start 16.379137 7.079137) (mid 15.96661 7.354779) (end 15.48 7.451572) (width 0.2) (layer "F.Cu") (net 5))
 (arc (start 27.75 7.02) (mid 27.867157 6.737157) (end 28.15 6.62) (width 0.2) (layer "F.Cu") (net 5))
 (arc (start 28.75 7.02) (mid 28.632843 6.737157) (end 28.35 6.62) (width 0.2) (layer "F.Cu") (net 5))
 (arc (start 24.9 9.8) (mid 24.593854 9.739104) (end 24.334315 9.565686) (width 0.2) (layer "F.Cu") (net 5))
 (arc (start 12.2 6.18) (mid 12.572435 7.079137) (end 13.471572 7.451572) (width 0.2) (layer "F.Cu") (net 5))
 (arc (start 19.65 5.5) (mid 19.503553 5.853553) (end 19.15 6) (width 0.2) (layer "F.Cu") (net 5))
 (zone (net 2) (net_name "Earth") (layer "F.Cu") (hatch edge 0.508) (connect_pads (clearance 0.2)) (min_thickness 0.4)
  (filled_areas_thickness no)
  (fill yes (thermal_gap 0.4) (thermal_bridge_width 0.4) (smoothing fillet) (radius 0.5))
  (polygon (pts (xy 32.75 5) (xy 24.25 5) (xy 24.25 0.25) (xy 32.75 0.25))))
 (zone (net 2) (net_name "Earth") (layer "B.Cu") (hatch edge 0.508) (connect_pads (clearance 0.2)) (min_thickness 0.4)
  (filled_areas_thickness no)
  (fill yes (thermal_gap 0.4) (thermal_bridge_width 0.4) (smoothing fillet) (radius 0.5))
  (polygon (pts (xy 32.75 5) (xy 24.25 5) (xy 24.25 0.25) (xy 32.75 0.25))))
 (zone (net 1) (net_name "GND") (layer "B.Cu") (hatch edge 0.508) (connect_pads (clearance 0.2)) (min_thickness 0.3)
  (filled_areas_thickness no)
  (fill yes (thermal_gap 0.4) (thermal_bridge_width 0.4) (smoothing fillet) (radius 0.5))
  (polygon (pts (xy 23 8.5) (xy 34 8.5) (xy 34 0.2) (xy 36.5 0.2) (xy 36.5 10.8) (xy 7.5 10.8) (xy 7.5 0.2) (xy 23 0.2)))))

